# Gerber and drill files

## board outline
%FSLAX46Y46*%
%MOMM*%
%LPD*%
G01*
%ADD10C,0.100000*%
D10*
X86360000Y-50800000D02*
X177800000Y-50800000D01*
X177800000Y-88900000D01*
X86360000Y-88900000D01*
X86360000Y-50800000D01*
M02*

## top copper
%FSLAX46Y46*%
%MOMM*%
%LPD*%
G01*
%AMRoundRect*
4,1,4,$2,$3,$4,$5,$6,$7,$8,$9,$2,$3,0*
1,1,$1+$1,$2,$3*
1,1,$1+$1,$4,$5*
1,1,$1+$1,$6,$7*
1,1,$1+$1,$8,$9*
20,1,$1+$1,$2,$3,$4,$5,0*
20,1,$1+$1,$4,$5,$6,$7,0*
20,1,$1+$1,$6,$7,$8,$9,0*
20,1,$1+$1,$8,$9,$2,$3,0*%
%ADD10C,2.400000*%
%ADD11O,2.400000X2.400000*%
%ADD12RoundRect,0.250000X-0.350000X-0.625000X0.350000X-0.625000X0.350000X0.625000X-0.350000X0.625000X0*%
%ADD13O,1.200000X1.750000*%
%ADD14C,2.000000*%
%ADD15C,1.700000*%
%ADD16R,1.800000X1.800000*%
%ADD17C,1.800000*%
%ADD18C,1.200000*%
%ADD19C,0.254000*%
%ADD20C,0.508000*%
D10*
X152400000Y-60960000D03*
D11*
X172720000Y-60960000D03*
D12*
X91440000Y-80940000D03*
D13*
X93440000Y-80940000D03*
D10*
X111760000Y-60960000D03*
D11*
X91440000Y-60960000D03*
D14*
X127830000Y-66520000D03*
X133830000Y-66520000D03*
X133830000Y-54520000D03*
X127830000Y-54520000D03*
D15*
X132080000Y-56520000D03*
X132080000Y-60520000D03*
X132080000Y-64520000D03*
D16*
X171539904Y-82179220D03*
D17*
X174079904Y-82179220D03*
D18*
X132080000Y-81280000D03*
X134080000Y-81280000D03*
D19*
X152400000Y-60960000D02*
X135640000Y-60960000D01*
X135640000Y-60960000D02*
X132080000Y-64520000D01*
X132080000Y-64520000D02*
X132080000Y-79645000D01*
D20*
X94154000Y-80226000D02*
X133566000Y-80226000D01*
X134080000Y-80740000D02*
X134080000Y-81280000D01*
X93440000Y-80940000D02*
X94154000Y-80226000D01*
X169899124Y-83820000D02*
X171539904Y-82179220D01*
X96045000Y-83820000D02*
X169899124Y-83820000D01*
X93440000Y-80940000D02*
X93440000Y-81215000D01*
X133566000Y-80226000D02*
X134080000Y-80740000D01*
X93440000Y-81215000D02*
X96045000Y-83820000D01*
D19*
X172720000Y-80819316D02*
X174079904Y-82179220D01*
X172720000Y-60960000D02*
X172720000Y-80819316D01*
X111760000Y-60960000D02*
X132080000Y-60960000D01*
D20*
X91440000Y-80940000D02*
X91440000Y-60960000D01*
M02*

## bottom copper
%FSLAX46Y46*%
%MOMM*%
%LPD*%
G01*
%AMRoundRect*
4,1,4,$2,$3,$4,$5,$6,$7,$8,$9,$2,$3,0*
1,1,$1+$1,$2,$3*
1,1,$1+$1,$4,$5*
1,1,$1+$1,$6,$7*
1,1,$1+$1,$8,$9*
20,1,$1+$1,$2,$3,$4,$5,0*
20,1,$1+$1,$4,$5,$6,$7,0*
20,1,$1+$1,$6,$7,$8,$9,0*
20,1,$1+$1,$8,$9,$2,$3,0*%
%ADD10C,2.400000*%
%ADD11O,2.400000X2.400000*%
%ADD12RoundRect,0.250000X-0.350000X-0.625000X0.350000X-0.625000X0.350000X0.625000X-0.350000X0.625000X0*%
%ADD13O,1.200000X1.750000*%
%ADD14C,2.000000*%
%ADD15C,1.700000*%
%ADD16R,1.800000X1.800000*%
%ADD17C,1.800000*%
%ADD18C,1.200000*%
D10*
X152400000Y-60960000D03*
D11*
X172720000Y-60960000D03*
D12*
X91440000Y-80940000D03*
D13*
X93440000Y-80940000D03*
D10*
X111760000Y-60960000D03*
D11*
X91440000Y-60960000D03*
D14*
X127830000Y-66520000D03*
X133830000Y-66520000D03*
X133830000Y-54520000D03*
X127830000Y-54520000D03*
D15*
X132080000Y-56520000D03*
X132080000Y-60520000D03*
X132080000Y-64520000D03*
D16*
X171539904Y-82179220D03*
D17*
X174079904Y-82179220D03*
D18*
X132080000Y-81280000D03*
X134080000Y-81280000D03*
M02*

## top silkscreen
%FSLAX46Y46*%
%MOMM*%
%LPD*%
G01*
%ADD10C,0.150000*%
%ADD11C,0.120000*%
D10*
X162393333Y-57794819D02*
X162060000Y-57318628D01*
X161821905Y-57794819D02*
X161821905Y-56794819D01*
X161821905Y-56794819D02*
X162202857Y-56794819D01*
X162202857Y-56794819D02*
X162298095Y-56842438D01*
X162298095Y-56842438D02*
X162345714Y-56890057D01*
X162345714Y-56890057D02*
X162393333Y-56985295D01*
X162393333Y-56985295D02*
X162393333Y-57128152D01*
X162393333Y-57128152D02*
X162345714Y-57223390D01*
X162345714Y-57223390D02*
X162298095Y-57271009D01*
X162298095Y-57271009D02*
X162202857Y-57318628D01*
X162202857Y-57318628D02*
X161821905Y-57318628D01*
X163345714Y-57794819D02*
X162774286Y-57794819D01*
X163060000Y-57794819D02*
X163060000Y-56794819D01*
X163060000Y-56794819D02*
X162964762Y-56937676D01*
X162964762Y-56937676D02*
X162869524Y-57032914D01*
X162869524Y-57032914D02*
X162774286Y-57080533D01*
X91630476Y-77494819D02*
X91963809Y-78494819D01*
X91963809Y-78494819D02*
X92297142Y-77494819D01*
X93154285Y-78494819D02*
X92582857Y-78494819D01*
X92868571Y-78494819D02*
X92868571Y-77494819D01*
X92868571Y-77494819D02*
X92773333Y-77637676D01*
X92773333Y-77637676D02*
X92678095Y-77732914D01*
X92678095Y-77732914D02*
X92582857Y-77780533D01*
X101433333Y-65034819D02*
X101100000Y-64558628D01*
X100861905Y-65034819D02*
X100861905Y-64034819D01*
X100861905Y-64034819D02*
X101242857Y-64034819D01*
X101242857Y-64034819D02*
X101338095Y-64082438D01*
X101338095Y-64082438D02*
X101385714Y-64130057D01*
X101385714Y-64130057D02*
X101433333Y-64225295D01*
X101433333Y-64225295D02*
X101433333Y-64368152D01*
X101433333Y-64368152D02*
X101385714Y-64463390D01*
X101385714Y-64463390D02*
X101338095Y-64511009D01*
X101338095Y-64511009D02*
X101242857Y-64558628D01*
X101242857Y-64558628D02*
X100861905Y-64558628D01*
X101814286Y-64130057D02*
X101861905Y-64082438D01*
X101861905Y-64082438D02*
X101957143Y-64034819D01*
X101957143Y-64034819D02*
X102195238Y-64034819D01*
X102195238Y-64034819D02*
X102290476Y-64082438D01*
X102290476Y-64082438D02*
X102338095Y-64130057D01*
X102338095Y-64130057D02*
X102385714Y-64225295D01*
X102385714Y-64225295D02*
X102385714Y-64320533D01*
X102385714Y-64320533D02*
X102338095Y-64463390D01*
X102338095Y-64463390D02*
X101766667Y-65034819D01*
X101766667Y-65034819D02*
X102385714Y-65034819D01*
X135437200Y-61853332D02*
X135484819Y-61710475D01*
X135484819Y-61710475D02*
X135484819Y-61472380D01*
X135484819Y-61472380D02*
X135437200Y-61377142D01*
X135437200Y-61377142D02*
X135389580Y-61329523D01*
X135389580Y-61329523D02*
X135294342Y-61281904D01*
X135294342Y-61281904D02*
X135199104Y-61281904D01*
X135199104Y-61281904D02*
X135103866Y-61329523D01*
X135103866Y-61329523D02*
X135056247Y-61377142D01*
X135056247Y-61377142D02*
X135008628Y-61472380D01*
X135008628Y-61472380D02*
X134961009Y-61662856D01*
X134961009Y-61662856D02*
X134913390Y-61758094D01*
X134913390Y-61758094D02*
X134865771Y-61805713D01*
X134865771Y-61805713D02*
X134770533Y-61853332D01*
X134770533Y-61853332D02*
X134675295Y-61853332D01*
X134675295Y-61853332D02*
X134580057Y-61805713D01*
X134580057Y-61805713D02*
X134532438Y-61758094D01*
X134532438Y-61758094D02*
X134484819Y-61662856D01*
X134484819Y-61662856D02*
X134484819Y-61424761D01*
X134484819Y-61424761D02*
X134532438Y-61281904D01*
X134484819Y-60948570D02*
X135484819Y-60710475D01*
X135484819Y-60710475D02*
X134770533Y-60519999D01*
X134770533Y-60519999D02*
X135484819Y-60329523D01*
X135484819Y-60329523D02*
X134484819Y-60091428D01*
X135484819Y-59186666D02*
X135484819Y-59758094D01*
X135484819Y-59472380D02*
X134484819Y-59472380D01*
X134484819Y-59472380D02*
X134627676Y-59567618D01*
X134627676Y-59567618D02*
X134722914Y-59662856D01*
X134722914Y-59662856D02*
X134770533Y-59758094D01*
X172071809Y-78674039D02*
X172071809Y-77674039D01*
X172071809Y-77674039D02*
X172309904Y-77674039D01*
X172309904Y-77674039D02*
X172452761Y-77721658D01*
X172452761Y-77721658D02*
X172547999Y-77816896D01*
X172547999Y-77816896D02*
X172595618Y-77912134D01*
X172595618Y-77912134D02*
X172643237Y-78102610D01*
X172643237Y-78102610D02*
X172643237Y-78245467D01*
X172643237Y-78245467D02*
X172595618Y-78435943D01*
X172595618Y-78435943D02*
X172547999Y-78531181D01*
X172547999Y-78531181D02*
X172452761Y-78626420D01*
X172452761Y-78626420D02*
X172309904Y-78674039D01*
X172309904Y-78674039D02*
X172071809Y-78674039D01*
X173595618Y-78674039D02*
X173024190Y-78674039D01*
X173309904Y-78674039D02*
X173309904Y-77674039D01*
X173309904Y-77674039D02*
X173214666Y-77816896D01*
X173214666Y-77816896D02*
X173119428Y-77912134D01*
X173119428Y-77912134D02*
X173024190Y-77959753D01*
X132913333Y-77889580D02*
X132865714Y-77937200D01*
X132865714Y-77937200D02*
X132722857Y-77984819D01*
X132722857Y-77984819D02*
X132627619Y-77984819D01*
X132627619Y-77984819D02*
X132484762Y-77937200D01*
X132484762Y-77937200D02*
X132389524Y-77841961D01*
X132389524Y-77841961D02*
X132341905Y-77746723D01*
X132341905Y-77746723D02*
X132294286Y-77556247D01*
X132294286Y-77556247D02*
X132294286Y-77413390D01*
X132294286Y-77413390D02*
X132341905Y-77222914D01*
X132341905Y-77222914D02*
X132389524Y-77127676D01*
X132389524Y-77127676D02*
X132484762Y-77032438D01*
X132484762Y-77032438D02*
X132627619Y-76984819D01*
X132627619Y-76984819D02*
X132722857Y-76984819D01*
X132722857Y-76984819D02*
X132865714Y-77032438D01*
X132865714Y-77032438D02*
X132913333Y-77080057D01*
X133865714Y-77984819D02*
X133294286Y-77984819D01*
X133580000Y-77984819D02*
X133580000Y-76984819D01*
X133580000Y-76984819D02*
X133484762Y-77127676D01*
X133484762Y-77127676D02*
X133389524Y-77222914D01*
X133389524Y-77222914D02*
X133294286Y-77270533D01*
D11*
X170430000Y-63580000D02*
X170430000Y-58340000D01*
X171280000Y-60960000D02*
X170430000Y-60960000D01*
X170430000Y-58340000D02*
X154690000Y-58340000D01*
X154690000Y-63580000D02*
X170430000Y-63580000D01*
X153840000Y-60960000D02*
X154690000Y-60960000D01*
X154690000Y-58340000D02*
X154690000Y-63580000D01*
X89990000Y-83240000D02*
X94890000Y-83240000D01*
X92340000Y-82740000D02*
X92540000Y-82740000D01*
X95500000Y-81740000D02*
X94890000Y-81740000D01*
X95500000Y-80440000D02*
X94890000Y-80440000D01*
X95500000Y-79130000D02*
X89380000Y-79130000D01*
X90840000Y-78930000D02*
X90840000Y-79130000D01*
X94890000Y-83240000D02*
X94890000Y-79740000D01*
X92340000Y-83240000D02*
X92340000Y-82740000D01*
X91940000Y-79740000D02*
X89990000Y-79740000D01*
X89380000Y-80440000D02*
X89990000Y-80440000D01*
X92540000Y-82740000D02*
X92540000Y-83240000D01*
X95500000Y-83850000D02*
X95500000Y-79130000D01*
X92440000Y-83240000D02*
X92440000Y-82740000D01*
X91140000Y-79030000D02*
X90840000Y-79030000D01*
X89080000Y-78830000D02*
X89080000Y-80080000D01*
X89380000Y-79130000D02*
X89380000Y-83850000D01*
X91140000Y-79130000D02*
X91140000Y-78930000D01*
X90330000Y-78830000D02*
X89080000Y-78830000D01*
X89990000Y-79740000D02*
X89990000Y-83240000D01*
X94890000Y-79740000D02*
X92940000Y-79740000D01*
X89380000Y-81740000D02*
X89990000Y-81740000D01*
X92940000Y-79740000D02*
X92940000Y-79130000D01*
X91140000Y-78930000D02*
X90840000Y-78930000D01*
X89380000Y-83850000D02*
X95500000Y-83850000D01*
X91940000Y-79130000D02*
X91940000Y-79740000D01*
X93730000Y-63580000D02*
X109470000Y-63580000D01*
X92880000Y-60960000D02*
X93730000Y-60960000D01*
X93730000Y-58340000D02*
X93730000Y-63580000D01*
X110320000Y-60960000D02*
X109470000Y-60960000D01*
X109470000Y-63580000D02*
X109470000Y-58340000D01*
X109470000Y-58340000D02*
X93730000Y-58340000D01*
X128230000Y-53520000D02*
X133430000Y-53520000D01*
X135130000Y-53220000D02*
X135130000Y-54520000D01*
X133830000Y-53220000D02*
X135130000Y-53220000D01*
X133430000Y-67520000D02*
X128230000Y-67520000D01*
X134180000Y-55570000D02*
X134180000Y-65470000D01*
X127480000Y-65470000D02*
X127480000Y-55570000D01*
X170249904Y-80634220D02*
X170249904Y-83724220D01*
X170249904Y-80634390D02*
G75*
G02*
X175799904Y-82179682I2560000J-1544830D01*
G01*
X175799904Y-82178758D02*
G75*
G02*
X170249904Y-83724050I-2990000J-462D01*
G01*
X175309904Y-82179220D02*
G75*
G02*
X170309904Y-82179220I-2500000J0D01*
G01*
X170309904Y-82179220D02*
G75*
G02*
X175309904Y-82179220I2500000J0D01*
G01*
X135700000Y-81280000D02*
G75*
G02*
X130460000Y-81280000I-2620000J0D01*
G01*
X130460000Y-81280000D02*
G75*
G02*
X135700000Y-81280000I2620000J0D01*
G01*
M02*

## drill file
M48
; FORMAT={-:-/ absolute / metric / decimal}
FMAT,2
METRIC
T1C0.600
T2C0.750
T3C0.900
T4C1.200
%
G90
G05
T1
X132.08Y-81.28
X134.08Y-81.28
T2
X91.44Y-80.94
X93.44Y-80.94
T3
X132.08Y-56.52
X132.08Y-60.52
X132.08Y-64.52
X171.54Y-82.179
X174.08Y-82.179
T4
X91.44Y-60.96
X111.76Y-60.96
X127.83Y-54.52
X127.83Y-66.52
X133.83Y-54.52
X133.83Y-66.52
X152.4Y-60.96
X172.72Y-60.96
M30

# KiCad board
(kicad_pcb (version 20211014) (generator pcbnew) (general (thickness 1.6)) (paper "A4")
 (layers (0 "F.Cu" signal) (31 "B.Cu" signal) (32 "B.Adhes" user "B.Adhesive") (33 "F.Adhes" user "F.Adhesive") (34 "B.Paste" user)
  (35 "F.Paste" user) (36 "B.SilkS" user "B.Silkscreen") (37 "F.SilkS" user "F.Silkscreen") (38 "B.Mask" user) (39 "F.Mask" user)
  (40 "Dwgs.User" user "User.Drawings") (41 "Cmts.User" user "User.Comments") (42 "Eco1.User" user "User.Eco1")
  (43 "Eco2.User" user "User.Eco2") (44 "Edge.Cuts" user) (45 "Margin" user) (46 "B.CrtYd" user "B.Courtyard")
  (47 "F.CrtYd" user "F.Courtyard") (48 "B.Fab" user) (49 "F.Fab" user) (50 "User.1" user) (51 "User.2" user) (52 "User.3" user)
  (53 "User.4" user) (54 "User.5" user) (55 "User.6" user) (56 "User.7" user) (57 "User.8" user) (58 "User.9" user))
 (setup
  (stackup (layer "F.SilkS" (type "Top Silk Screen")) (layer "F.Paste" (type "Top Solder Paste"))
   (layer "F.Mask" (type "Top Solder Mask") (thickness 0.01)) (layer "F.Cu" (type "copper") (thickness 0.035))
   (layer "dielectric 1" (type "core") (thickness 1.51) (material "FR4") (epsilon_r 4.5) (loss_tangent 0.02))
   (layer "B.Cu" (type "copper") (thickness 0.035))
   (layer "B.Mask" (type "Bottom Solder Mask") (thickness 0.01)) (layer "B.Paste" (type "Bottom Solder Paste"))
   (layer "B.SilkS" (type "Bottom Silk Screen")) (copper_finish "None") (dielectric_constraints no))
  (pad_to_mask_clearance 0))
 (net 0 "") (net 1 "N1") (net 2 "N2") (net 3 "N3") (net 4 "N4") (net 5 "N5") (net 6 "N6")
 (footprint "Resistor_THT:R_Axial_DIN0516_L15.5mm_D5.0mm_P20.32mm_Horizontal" (layer "F.Cu") (at 152.4 60.96)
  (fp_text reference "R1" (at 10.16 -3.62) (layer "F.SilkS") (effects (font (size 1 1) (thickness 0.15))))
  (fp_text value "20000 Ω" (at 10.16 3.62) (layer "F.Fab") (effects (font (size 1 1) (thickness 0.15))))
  (fp_line (start 18.03 2.62) (end 18.03 -2.62) (layer "F.SilkS") (width 0.12))
  (fp_line (start 18.88 0) (end 18.03 0) (layer "F.SilkS") (width 0.12))
  (fp_line (start 18.03 -2.62) (end 2.29 -2.62) (layer "F.SilkS") (width 0.12))
  (fp_line (start 2.29 2.62) (end 18.03 2.62) (layer "F.SilkS") (width 0.12))
  (fp_line (start 1.44 0) (end 2.29 0) (layer "F.SilkS") (width 0.12))
  (fp_line (start 2.29 -2.62) (end 2.29 2.62) (layer "F.SilkS") (width 0.12))
  (pad "1" thru_hole circle (at 0 0) (size 2.4 2.4) (drill 1.2) (layers *.Cu *.Mask) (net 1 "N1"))
  (pad "2" thru_hole oval (at 20.32 0) (size 2.4 2.4) (drill 1.2) (layers *.Cu *.Mask) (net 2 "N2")))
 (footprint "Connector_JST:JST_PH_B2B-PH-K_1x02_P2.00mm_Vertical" (layer "F.Cu") (at 91.44 80.94)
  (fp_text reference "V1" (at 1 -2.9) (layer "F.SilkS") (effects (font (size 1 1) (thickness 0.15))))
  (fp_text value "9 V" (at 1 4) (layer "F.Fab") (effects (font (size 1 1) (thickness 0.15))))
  (fp_line (start -1.45 2.3) (end 3.45 2.3) (layer "F.SilkS") (width 0.12))
  (fp_line (start 0.9 1.8) (end 1.1 1.8) (layer "F.SilkS") (width 0.12))
  (fp_line (start 4.06 0.8) (end 3.45 0.8) (layer "F.SilkS") (width 0.12))
  (fp_line (start 4.06 -0.5) (end 3.45 -0.5) (layer "F.SilkS") (width 0.12))
  (fp_line (start 4.06 -1.81) (end -2.06 -1.81) (layer "F.SilkS") (width 0.12))
  (fp_line (start -0.6 -2.01) (end -0.6 -1.81) (layer "F.SilkS") (width 0.12))
  (fp_line (start 3.45 2.3) (end 3.45 -1.2) (layer "F.SilkS") (width 0.12))
  (fp_line (start 0.9 2.3) (end 0.9 1.8) (layer "F.SilkS") (width 0.12))
  (fp_line (start 0.5 -1.2) (end -1.45 -1.2) (layer "F.SilkS") (width 0.12))
  (fp_line (start -2.06 -0.5) (end -1.45 -0.5) (layer "F.SilkS") (width 0.12))
  (fp_line (start 1.1 1.8) (end 1.1 2.3) (layer "F.SilkS") (width 0.12))
  (fp_line (start 4.06 2.91) (end 4.06 -1.81) (layer "F.SilkS") (width 0.12))
  (fp_line (start 1 2.3) (end 1 1.8) (layer "F.SilkS") (width 0.12))
  (fp_line (start -0.3 -1.91) (end -0.6 -1.91) (layer "F.SilkS") (width 0.12))
  (fp_line (start -2.36 -2.11) (end -2.36 -0.86) (layer "F.SilkS") (width 0.12))
  (fp_line (start -2.06 -1.81) (end -2.06 2.91) (layer "F.SilkS") (width 0.12))
  (fp_line (start -0.3 -1.81) (end -0.3 -2.01) (layer "F.SilkS") (width 0.12))
  (fp_line (start -1.11 -2.11) (end -2.36 -2.11) (layer "F.SilkS") (width 0.12))
  (fp_line (start -1.45 -1.2) (end -1.45 2.3) (layer "F.SilkS") (width 0.12))
  (fp_line (start 3.45 -1.2) (end 1.5 -1.2) (layer "F.SilkS") (width 0.12))
  (fp_line (start -2.06 0.8) (end -1.45 0.8) (layer "F.SilkS") (width 0.12))
  (fp_line (start 1.5 -1.2) (end 1.5 -1.81) (layer "F.SilkS") (width 0.12))
  (fp_line (start -0.3 -2.01) (end -0.6 -2.01) (layer "F.SilkS") (width 0.12))
  (fp_line (start -2.06 2.91) (end 4.06 2.91) (layer "F.SilkS") (width 0.12))
  (fp_line (start 0.5 -1.81) (end 0.5 -1.2) (layer "F.SilkS") (width 0.12))
  (pad "1" thru_hole roundrect (at 0 0) (size 1.2 1.75) (drill 0.75) (layers *.Cu *.Mask) (roundrect_rratio 0.208333) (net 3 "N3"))
  (pad "2" thru_hole oval (at 2 0) (size 1.2 1.75) (drill 0.75) (layers *.Cu *.Mask) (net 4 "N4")))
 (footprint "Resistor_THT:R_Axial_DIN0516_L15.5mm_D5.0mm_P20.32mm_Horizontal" (layer "F.Cu") (at 111.76 60.96 180)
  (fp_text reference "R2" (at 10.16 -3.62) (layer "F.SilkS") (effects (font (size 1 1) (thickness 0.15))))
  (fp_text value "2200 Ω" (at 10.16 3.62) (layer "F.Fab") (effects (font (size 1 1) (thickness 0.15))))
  (fp_line (start 18.03 -2.62) (end 2.29 -2.62) (layer "F.SilkS") (width 0.12))
  (fp_line (start 18.88 0) (end 18.03 0) (layer "F.SilkS") (width 0.12))
  (fp_line (start 18.03 2.62) (end 18.03 -2.62) (layer "F.SilkS") (width 0.12))
  (fp_line (start 1.44 0) (end 2.29 0) (layer "F.SilkS") (width 0.12))
  (fp_line (start 2.29 -2.62) (end 2.29 2.62) (layer "F.SilkS") (width 0.12))
  (fp_line (start 2.29 2.62) (end 18.03 2.62) (layer "F.SilkS") (width 0.12))
  (pad "1" thru_hole circle (at 0 0 180) (size 2.4 2.4) (drill 1.2) (layers *.Cu *.Mask) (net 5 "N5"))
  (pad "2" thru_hole oval (at 20.32 0 180) (size 2.4 2.4) (drill 1.2) (layers *.Cu *.Mask) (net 3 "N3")))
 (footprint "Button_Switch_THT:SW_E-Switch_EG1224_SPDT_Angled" (layer "F.Cu") (at 132.08 56.52 -90)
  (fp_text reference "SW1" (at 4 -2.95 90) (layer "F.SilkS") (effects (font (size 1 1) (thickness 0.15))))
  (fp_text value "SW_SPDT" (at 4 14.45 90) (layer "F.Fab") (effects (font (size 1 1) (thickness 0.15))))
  (fp_line (start -3 3.85) (end -3 -1.35) (layer "F.SilkS") (width 0.12))
  (fp_line (start -3.3 -3.05) (end -2 -3.05) (layer "F.SilkS") (width 0.12))
  (fp_line (start -3.3 -1.75) (end -3.3 -3.05) (layer "F.SilkS") (width 0.12))
  (fp_line (start 11 -1.35) (end 11 3.85) (layer "F.SilkS") (width 0.12))
  (fp_line (start -0.95 -2.1) (end 8.95 -2.1) (layer "F.SilkS") (width 0.12))
  (fp_line (start 8.95 4.6) (end -0.95 4.6) (layer "F.SilkS") (width 0.12))
  (pad "" thru_hole circle (at 10 4.25 270) (size 2 2) (drill 1.2) (layers *.Cu *.Mask))
  (pad "" thru_hole circle (at 10 -1.75 270) (size 2 2) (drill 1.2) (layers *.Cu *.Mask))
  (pad "" thru_hole circle (at -2 -1.75 270) (size 2 2) (drill 1.2) (layers *.Cu *.Mask))
  (pad "" thru_hole circle (at -2 4.25 270) (size 2 2) (drill 1.2) (layers *.Cu *.Mask))
  (pad "1" thru_hole circle (at 0 0 270) (size 1.7 1.7) (drill 0.9) (layers *.Cu *.Mask) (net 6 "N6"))
  (pad "2" thru_hole circle (at 4 0 270) (size 1.7 1.7) (drill 0.9) (layers *.Cu *.Mask) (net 5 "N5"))
  (pad "3" thru_hole circle (at 8 0 270) (size 1.7 1.7) (drill 0.9) (layers *.Cu *.Mask) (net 1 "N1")))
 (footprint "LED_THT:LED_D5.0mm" (layer "F.Cu") (at 171.539904 82.17922)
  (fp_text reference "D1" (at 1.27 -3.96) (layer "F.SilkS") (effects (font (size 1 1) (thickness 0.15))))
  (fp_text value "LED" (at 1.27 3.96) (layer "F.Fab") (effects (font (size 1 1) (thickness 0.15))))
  (fp_line (start -1.29 -1.545) (end -1.29 1.545) (layer "F.SilkS") (width 0.12))
  (fp_arc (start -1.29 -1.54483) (mid 2.072002 -2.880433) (end 4.26 0.000462) (layer "F.SilkS") (width 0.12))
  (fp_arc (start 4.26 -0.000462) (mid 2.072002 2.880433) (end -1.29 1.54483) (layer "F.SilkS") (width 0.12))
  (fp_circle (center 1.27 0) (end 3.77 0) (layer "F.SilkS") (width 0.12) (fill none))
  (pad "1" thru_hole rect (at 0 0) (size 1.8 1.8) (drill 0.9) (layers *.Cu *.Mask) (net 4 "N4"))
  (pad "2" thru_hole circle (at 2.54 0) (size 1.8 1.8) (drill 0.9) (layers *.Cu *.Mask) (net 2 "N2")))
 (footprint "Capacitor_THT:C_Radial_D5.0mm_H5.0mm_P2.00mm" (layer "F.Cu") (at 132.08 81.28)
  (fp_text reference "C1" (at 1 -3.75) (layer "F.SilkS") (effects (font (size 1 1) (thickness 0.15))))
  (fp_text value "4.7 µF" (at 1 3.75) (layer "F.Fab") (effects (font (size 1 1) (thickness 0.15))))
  (fp_circle (center 1 0) (end 3.62 0) (layer "F.SilkS") (width 0.12) (fill none))
  (pad "1" thru_hole circle (at 0 0) (size 1.2 1.2) (drill 0.6) (layers *.Cu *.Mask) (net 1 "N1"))
  (pad "2" thru_hole circle (at 2 0) (size 1.2 1.2) (drill 0.6) (layers *.Cu *.Mask) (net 4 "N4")))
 (gr_rect (start 86.36 50.8) (end 177.8 88.9) (layer "Edge.Cuts") (width 0.1) (fill none))
 (segment (start 152.4 60.96) (end 135.64 60.96) (width 0.254) (layer "F.Cu") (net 1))
 (segment (start 135.64 60.96) (end 132.08 64.52) (width 0.254) (layer "F.Cu") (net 1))
 (segment (start 132.08 64.52) (end 132.08 79.645) (width 0.254) (layer "F.Cu") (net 1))
 (segment (start 94.154 80.226) (end 133.566 80.226) (width 0.508) (layer "F.Cu") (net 4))
 (segment (start 134.08 80.74) (end 134.08 81.28) (width 0.508) (layer "F.Cu") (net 4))
 (segment (start 93.44 80.94) (end 94.154 80.226) (width 0.508) (layer "F.Cu") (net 4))
 (segment (start 169.899124 83.82) (end 171.539904 82.17922) (width 0.508) (layer "F.Cu") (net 4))
 (segment (start 96.045 83.82) (end 169.899124 83.82) (width 0.508) (layer "F.Cu") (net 4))
 (segment (start 93.44 80.94) (end 93.44 81.215) (width 0.508) (layer "F.Cu") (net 4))
 (segment (start 133.566 80.226) (end 134.08 80.74) (width 0.508) (layer "F.Cu") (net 4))
 (segment (start 93.44 81.215) (end 96.045 83.82) (width 0.508) (layer "F.Cu") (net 4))
 (segment (start 172.72 80.819316) (end 174.079904 82.17922) (width 0.254) (layer "F.Cu") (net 2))
 (segment (start 172.72 60.96) (end 172.72 80.819316) (width 0.254) (layer "F.Cu") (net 2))
 (segment (start 111.76 60.96) (end 132.08 60.96) (width 0.254) (layer "F.Cu") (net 5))
 (segment (start 91.44 80.94) (end 91.44 60.96) (width 0.508) (layer "F.Cu") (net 3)))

